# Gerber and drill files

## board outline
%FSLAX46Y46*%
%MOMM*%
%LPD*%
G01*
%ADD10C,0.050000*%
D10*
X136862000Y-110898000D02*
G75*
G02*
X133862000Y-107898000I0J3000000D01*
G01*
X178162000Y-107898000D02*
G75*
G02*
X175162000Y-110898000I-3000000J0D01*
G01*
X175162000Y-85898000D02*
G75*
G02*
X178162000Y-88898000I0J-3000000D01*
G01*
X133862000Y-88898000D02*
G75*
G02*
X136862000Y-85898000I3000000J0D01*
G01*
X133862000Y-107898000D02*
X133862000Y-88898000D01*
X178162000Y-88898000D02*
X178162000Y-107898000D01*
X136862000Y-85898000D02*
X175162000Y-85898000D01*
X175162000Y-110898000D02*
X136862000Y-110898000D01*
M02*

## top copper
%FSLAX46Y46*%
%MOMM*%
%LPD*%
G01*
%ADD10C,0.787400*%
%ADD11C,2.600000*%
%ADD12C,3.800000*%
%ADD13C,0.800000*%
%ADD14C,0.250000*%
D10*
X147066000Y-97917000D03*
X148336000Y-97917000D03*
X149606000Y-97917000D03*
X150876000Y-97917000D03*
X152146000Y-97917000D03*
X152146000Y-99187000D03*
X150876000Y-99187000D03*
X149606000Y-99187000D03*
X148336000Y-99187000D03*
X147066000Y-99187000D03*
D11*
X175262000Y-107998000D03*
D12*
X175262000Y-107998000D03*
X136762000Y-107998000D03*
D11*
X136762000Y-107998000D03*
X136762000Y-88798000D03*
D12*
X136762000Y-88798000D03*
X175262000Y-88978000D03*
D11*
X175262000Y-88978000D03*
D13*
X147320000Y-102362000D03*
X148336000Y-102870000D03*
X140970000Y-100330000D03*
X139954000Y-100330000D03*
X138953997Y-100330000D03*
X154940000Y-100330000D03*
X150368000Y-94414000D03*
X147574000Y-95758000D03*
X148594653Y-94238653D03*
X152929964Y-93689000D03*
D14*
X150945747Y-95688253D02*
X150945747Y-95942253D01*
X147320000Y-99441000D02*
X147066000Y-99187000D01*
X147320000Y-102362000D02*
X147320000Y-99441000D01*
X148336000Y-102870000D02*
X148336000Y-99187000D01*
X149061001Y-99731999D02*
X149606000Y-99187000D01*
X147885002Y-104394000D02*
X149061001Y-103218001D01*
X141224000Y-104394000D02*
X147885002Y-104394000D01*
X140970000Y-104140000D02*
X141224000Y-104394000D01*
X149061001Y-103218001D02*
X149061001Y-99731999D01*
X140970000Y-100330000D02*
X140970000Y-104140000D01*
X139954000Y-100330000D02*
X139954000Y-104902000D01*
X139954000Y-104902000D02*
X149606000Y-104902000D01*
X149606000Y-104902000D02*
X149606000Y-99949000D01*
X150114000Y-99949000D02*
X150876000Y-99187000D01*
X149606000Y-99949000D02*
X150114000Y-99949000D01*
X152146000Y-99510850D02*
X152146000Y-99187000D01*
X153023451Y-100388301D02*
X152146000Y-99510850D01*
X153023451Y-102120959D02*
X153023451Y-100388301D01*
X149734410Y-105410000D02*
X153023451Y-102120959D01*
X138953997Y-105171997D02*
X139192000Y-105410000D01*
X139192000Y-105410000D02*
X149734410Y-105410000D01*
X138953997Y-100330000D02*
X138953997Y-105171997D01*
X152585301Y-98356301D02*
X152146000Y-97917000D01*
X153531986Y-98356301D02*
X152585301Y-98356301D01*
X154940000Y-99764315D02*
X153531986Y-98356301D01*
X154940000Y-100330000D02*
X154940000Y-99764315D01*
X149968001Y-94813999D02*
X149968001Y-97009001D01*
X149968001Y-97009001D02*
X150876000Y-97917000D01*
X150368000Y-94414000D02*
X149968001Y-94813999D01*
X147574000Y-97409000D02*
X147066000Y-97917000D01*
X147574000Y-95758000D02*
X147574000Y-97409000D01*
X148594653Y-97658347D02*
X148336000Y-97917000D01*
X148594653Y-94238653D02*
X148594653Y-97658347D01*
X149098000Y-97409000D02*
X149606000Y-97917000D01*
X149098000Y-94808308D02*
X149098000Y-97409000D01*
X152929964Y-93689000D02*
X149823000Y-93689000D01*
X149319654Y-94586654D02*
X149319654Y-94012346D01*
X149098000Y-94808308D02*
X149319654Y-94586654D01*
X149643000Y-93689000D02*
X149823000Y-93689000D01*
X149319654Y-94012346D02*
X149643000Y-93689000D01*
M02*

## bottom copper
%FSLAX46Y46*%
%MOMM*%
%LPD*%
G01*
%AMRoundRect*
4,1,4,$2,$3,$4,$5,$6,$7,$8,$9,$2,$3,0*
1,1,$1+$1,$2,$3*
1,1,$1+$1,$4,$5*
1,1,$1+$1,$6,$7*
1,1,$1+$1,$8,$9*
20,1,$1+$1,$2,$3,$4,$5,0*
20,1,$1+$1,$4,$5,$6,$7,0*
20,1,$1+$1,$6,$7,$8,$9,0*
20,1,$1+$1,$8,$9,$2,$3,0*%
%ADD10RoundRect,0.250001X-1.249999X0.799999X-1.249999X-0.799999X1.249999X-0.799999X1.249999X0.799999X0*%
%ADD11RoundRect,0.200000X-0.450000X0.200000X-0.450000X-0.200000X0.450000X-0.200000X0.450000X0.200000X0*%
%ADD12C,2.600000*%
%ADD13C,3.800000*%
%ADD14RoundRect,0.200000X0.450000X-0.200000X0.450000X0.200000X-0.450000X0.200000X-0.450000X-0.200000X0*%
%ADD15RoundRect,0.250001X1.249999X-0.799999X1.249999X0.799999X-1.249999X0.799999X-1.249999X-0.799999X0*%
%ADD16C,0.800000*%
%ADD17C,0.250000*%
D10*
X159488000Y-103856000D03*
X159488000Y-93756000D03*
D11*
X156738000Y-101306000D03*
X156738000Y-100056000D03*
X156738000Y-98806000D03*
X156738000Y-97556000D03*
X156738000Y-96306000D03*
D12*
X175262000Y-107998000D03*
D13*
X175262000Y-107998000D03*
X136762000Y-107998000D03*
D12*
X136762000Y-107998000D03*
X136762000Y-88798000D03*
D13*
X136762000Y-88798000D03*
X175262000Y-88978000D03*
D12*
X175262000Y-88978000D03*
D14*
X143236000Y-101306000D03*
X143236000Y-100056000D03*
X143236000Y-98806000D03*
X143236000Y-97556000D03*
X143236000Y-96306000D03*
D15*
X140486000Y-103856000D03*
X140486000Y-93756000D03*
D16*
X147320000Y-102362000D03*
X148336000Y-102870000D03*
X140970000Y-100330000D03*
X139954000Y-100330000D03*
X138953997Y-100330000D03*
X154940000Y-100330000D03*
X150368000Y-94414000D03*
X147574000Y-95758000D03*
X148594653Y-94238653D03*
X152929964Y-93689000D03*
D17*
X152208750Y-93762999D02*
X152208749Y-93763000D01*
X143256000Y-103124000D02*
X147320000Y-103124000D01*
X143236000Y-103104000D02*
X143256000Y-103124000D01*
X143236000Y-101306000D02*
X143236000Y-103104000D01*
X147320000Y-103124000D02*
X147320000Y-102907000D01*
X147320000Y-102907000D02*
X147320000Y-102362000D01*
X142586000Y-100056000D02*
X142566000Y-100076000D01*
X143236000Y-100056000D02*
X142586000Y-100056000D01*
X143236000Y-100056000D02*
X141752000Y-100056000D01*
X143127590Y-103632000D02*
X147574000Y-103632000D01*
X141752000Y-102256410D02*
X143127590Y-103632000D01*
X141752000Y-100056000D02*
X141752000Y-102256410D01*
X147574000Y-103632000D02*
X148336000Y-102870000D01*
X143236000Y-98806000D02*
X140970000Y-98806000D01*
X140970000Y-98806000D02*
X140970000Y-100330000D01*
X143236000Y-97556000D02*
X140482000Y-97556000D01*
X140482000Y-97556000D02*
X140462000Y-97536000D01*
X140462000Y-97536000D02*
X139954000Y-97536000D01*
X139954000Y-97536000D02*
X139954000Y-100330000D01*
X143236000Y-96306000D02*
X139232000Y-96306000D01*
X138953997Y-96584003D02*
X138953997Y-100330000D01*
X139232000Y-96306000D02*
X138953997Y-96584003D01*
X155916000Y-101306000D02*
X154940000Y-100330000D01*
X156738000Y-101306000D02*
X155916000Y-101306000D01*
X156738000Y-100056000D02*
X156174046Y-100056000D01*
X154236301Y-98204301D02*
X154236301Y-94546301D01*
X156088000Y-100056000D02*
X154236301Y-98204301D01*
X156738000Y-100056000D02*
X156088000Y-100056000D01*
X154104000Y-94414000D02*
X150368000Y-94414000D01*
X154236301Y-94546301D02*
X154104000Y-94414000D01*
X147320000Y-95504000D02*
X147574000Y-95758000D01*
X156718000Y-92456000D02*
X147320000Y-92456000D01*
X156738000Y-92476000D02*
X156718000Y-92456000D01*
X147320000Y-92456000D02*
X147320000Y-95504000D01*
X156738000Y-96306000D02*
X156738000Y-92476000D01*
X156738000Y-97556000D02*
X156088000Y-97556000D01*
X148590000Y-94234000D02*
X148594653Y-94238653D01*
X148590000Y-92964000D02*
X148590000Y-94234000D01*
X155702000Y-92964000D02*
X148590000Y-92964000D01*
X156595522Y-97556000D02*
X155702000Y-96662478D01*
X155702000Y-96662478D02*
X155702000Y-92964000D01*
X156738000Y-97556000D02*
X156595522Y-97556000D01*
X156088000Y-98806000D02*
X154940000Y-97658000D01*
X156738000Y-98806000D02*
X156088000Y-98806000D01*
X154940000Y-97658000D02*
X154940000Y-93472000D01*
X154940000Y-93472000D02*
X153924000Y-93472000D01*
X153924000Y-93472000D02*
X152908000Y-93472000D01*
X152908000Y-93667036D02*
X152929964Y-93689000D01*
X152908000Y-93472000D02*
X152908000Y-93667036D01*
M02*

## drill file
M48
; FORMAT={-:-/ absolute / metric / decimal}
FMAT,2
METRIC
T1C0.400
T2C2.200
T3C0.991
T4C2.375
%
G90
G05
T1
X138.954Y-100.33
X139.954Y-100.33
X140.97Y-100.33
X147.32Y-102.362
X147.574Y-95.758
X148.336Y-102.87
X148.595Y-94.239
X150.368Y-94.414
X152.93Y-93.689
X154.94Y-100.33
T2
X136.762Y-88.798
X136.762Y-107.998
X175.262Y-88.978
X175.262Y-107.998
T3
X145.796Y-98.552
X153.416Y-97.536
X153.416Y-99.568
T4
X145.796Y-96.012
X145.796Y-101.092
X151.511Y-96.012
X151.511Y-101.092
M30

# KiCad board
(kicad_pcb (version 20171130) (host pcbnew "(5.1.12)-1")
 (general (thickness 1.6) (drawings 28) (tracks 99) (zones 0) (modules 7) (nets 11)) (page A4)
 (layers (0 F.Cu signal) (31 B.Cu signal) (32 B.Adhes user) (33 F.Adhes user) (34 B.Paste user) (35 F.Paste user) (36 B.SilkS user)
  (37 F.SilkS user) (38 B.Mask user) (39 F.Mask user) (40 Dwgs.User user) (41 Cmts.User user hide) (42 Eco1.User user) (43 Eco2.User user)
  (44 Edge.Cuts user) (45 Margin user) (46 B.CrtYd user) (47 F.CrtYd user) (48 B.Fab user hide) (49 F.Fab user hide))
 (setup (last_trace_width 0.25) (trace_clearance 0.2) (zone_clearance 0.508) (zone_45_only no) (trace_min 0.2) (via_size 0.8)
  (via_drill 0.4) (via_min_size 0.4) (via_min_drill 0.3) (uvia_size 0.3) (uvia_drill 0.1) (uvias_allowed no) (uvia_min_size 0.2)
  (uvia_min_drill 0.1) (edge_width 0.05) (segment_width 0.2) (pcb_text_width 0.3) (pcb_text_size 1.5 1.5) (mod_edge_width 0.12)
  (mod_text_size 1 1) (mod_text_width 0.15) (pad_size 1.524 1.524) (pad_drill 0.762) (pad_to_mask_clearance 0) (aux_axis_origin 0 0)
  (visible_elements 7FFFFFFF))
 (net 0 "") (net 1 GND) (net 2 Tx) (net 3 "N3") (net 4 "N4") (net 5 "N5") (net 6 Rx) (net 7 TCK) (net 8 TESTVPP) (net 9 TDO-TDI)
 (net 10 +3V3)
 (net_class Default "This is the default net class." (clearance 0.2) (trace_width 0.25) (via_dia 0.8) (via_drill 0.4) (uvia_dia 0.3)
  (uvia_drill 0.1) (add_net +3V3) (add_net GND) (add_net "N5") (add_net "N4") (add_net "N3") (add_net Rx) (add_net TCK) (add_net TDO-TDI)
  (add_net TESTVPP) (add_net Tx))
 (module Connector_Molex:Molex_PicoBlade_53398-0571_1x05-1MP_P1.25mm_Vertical (layer B.Cu) (at 157.988 98.806 270)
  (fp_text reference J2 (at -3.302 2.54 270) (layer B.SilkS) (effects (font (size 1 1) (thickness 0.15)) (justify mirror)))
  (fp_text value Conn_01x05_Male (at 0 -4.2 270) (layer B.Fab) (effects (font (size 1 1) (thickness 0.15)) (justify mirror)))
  (pad MP smd roundrect (at 5.05 -1.5 270) (size 2.1 3) (layers B.Cu B.Paste B.Mask) (roundrect_rratio 0.119048))
  (pad MP smd roundrect (at -5.05 -1.5 270) (size 2.1 3) (layers B.Cu B.Paste B.Mask) (roundrect_rratio 0.119048))
  (pad 5 smd roundrect (at 2.5 1.25 270) (size 0.8 1.3) (layers B.Cu B.Paste B.Mask) (roundrect_rratio 0.25) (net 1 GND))
  (pad 4 smd roundrect (at 1.25 1.25 270) (size 0.8 1.3) (layers B.Cu B.Paste B.Mask) (roundrect_rratio 0.25) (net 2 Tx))
  (pad 3 smd roundrect (at 0 1.25 270) (size 0.8 1.3) (layers B.Cu B.Paste B.Mask) (roundrect_rratio 0.25) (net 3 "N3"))
  (pad 2 smd roundrect (at -1.25 1.25 270) (size 0.8 1.3) (layers B.Cu B.Paste B.Mask) (roundrect_rratio 0.25) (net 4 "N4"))
  (pad 1 smd roundrect (at -2.5 1.25 270) (size 0.8 1.3) (layers B.Cu B.Paste B.Mask) (roundrect_rratio 0.25) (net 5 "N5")))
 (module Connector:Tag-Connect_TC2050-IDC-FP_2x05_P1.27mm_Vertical (layer F.Cu) (at 149.606 98.552)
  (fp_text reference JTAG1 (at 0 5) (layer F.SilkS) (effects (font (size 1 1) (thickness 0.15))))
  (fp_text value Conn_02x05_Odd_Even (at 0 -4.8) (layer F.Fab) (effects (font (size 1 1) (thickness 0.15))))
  (pad "" np_thru_hole circle (at 1.905 -2.54) (size 2.3749 2.3749) (drill 2.3749) (layers *.Cu *.Mask))
  (pad "" np_thru_hole circle (at 1.905 2.54) (size 2.3749 2.3749) (drill 2.3749) (layers *.Cu *.Mask))
  (pad "" np_thru_hole circle (at -3.81 2.54) (size 2.3749 2.3749) (drill 2.3749) (layers *.Cu *.Mask))
  (pad "" np_thru_hole circle (at -3.81 -2.54) (size 2.3749 2.3749) (drill 2.3749) (layers *.Cu *.Mask))
  (pad 10 connect circle (at -2.54 -0.635) (size 0.7874 0.7874) (layers F.Cu F.Mask) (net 5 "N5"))
  (pad 9 connect circle (at -1.27 -0.635) (size 0.7874 0.7874) (layers F.Cu F.Mask) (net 4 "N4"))
  (pad 8 connect circle (at 0 -0.635) (size 0.7874 0.7874) (layers F.Cu F.Mask) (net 3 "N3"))
  (pad 7 connect circle (at 1.27 -0.635) (size 0.7874 0.7874) (layers F.Cu F.Mask) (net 2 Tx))
  (pad 6 connect circle (at 2.54 -0.635) (size 0.7874 0.7874) (layers F.Cu F.Mask) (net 1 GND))
  (pad 5 connect circle (at 2.54 0.635) (size 0.7874 0.7874) (layers F.Cu F.Mask) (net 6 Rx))
  (pad 4 connect circle (at 1.27 0.635) (size 0.7874 0.7874) (layers F.Cu F.Mask) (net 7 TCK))
  (pad 3 connect circle (at 0 0.635) (size 0.7874 0.7874) (layers F.Cu F.Mask) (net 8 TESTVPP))
  (pad 2 connect circle (at -1.27 0.635) (size 0.7874 0.7874) (layers F.Cu F.Mask) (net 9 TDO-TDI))
  (pad 1 connect circle (at -2.54 0.635) (size 0.7874 0.7874) (layers F.Cu F.Mask) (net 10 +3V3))
  (pad "" np_thru_hole circle (at -3.81 0) (size 0.9906 0.9906) (drill 0.9906) (layers *.Cu *.Mask))
  (pad "" np_thru_hole circle (at 3.81 1.016) (size 0.9906 0.9906) (drill 0.9906) (layers *.Cu *.Mask))
  (pad "" np_thru_hole circle (at 3.81 -1.016) (size 0.9906 0.9906) (drill 0.9906) (layers *.Cu *.Mask)))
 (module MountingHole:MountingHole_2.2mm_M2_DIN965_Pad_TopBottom (layer F.Cu) (at 175.262 107.998)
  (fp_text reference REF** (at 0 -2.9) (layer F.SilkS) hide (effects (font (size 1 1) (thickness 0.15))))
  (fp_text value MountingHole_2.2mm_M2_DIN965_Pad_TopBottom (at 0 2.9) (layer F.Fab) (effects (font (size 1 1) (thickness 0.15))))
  (pad 1 thru_hole circle (at 0 0) (size 2.6 2.6) (drill 2.2) (layers *.Cu *.Mask))
  (pad 1 connect circle (at 0 0) (size 3.8 3.8) (layers F.Cu F.Mask))
  (pad 1 connect circle (at 0 0) (size 3.8 3.8) (layers B.Cu B.Mask)))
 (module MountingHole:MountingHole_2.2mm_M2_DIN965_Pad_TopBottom (layer F.Cu) (at 136.762 107.998)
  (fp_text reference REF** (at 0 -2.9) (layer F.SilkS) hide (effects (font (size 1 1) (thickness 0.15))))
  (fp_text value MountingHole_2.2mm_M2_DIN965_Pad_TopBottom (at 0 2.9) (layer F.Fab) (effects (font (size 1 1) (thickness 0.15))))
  (pad 1 connect circle (at 0 0) (size 3.8 3.8) (layers B.Cu B.Mask))
  (pad 1 connect circle (at 0 0) (size 3.8 3.8) (layers F.Cu F.Mask))
  (pad 1 thru_hole circle (at 0 0) (size 2.6 2.6) (drill 2.2) (layers *.Cu *.Mask)))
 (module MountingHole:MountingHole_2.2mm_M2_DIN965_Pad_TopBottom (layer F.Cu) (at 136.762 88.798)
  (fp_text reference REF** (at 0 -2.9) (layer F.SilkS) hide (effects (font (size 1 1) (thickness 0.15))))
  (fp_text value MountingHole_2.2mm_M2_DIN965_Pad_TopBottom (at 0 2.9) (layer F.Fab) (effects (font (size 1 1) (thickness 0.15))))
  (pad 1 thru_hole circle (at 0 0) (size 2.6 2.6) (drill 2.2) (layers *.Cu *.Mask))
  (pad 1 connect circle (at 0 0) (size 3.8 3.8) (layers F.Cu F.Mask))
  (pad 1 connect circle (at 0 0) (size 3.8 3.8) (layers B.Cu B.Mask)))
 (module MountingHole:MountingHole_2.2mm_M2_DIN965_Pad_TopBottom (layer F.Cu) (at 175.262 88.978)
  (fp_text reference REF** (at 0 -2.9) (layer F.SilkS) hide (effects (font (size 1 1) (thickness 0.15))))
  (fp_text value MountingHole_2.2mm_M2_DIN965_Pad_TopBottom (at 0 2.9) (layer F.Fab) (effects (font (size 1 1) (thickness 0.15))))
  (pad 1 connect circle (at 0 0) (size 3.8 3.8) (layers B.Cu B.Mask))
  (pad 1 connect circle (at 0 0) (size 3.8 3.8) (layers F.Cu F.Mask))
  (pad 1 thru_hole circle (at 0 0) (size 2.6 2.6) (drill 2.2) (layers *.Cu *.Mask)))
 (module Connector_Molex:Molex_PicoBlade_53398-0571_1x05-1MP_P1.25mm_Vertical (layer B.Cu) (at 141.986 98.806 90)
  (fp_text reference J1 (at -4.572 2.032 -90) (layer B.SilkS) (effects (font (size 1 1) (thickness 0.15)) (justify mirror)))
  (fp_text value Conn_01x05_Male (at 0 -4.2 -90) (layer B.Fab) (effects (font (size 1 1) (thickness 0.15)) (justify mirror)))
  (pad 1 smd roundrect (at -2.5 1.25 90) (size 0.8 1.3) (layers B.Cu B.Paste B.Mask) (roundrect_rratio 0.25) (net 10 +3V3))
  (pad 2 smd roundrect (at -1.25 1.25 90) (size 0.8 1.3) (layers B.Cu B.Paste B.Mask) (roundrect_rratio 0.25) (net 9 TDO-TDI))
  (pad 3 smd roundrect (at 0 1.25 90) (size 0.8 1.3) (layers B.Cu B.Paste B.Mask) (roundrect_rratio 0.25) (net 8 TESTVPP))
  (pad 4 smd roundrect (at 1.25 1.25 90) (size 0.8 1.3) (layers B.Cu B.Paste B.Mask) (roundrect_rratio 0.25) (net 7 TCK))
  (pad 5 smd roundrect (at 2.5 1.25 90) (size 0.8 1.3) (layers B.Cu B.Paste B.Mask) (roundrect_rratio 0.25) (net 6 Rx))
  (pad MP smd roundrect (at -5.05 -1.5 90) (size 2.1 3) (layers B.Cu B.Paste B.Mask) (roundrect_rratio 0.119048))
  (pad MP smd roundrect (at 5.05 -1.5 90) (size 2.1 3) (layers B.Cu B.Paste B.Mask) (roundrect_rratio 0.119048)))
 (gr_arc (start 136.862 107.898) (end 133.862 107.898) (angle -90) (layer Edge.Cuts) (width 0.05))
 (gr_arc (start 175.162 107.898) (end 175.162 110.898) (angle -90) (layer Edge.Cuts) (width 0.05))
 (gr_arc (start 175.162 88.898) (end 178.162 88.898) (angle -90) (layer Edge.Cuts) (width 0.05))
 (gr_arc (start 136.862 88.898) (end 136.862 85.898) (angle -90) (layer Edge.Cuts) (width 0.05))
 (gr_line (start 133.862 107.898) (end 133.862 88.898) (layer Edge.Cuts) (width 0.05))
 (gr_line (start 178.162 88.898) (end 178.162 107.898) (layer Edge.Cuts) (width 0.05))
 (gr_line (start 136.862 85.898) (end 175.162 85.898) (layer Edge.Cuts) (width 0.05))
 (gr_line (start 175.162 110.898) (end 136.862 110.898) (layer Edge.Cuts) (width 0.05))
 (segment (start 150.945747 95.688253) (end 150.945747 95.942253) (width 0.25) (layer F.Cu) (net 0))
 (segment (start 152.20875 93.762999) (end 152.208749 93.763) (width 0.25) (layer B.Cu) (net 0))
 (segment (start 143.256 103.124) (end 147.32 103.124) (width 0.25) (layer B.Cu) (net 10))
 (segment (start 143.236 103.104) (end 143.256 103.124) (width 0.25) (layer B.Cu) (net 10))
 (segment (start 143.236 101.306) (end 143.236 103.104) (width 0.25) (layer B.Cu) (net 10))
 (segment (start 147.32 103.124) (end 147.32 102.907) (width 0.25) (layer B.Cu) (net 10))
 (via (at 147.32 102.362) (size 0.8) (drill 0.4) (layers F.Cu B.Cu) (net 10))
 (segment (start 147.32 102.907) (end 147.32 102.362) (width 0.25) (layer B.Cu) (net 10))
 (segment (start 147.32 99.441) (end 147.066 99.187) (width 0.25) (layer F.Cu) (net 10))
 (segment (start 147.32 102.362) (end 147.32 99.441) (width 0.25) (layer F.Cu) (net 10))
 (segment (start 142.586 100.056) (end 142.566 100.076) (width 0.25) (layer B.Cu) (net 9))
 (segment (start 143.236 100.056) (end 142.586 100.056) (width 0.25) (layer B.Cu) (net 9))
 (segment (start 143.236 100.056) (end 141.752 100.056) (width 0.25) (layer B.Cu) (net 9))
 (segment (start 143.12759 103.632) (end 147.574 103.632) (width 0.25) (layer B.Cu) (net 9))
 (segment (start 141.752 102.25641) (end 143.12759 103.632) (width 0.25) (layer B.Cu) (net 9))
 (segment (start 141.752 100.056) (end 141.752 102.25641) (width 0.25) (layer B.Cu) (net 9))
 (via (at 148.336 102.87) (size 0.8) (drill 0.4) (layers F.Cu B.Cu) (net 9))
 (segment (start 147.574 103.632) (end 148.336 102.87) (width 0.25) (layer B.Cu) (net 9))
 (segment (start 148.336 102.87) (end 148.336 99.187) (width 0.25) (layer F.Cu) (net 9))
 (segment (start 143.236 98.806) (end 140.97 98.806) (width 0.25) (layer B.Cu) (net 8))
 (via (at 140.97 100.33) (size 0.8) (drill 0.4) (layers F.Cu B.Cu) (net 8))
 (segment (start 140.97 98.806) (end 140.97 100.33) (width 0.25) (layer B.Cu) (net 8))
 (segment (start 149.061001 99.731999) (end 149.606 99.187) (width 0.25) (layer F.Cu) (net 8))
 (segment (start 147.885002 104.394) (end 149.061001 103.218001) (width 0.25) (layer F.Cu) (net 8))
 (segment (start 141.224 104.394) (end 147.885002 104.394) (width 0.25) (layer F.Cu) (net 8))
 (segment (start 140.97 104.14) (end 141.224 104.394) (width 0.25) (layer F.Cu) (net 8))
 (segment (start 149.061001 103.218001) (end 149.061001 99.731999) (width 0.25) (layer F.Cu) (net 8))
 (segment (start 140.97 100.33) (end 140.97 104.14) (width 0.25) (layer F.Cu) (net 8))
 (segment (start 143.236 97.556) (end 140.482 97.556) (width 0.25) (layer B.Cu) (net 7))
 (segment (start 140.482 97.556) (end 140.462 97.536) (width 0.25) (layer B.Cu) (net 7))
 (segment (start 140.462 97.536) (end 139.954 97.536) (width 0.25) (layer B.Cu) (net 7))
 (via (at 139.954 100.33) (size 0.8) (drill 0.4) (layers F.Cu B.Cu) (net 7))
 (segment (start 139.954 97.536) (end 139.954 100.33) (width 0.25) (layer B.Cu) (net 7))
 (segment (start 139.954 100.33) (end 139.954 104.902) (width 0.25) (layer F.Cu) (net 7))
 (segment (start 139.954 104.902) (end 149.606 104.902) (width 0.25) (layer F.Cu) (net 7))
 (segment (start 149.606 104.902) (end 149.606 99.949) (width 0.25) (layer F.Cu) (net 7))
 (segment (start 150.114 99.949) (end 150.876 99.187) (width 0.25) (layer F.Cu) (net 7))
 (segment (start 149.606 99.949) (end 150.114 99.949) (width 0.25) (layer F.Cu) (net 7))
 (segment (start 143.236 96.306) (end 139.232 96.306) (width 0.25) (layer B.Cu) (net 6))
 (via (at 138.953997 100.33) (size 0.8) (drill 0.4) (layers F.Cu B.Cu) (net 6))
 (segment (start 138.953997 96.584003) (end 138.953997 100.33) (width 0.25) (layer B.Cu) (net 6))
 (segment (start 139.232 96.306) (end 138.953997 96.584003) (width 0.25) (layer B.Cu) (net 6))
 (segment (start 152.146 99.51085) (end 152.146 99.187) (width 0.25) (layer F.Cu) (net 6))
 (segment (start 153.023451 100.388301) (end 152.146 99.51085) (width 0.25) (layer F.Cu) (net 6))
 (segment (start 153.023451 102.120959) (end 153.023451 100.388301) (width 0.25) (layer F.Cu) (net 6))
 (segment (start 149.73441 105.41) (end 153.023451 102.120959) (width 0.25) (layer F.Cu) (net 6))
 (segment (start 138.953997 105.171997) (end 139.192 105.41) (width 0.25) (layer F.Cu) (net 6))
 (segment (start 139.192 105.41) (end 149.73441 105.41) (width 0.25) (layer F.Cu) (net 6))
 (segment (start 138.953997 100.33) (end 138.953997 105.171997) (width 0.25) (layer F.Cu) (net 6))
 (via (at 154.94 100.33) (size 0.8) (drill 0.4) (layers F.Cu B.Cu) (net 1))
 (segment (start 155.916 101.306) (end 154.94 100.33) (width 0.25) (layer B.Cu) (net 1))
 (segment (start 156.738 101.306) (end 155.916 101.306) (width 0.25) (layer B.Cu) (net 1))
 (segment (start 152.585301 98.356301) (end 152.146 97.917) (width 0.25) (layer F.Cu) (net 1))
 (segment (start 153.531986 98.356301) (end 152.585301 98.356301) (width 0.25) (layer F.Cu) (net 1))
 (segment (start 154.94 99.764315) (end 153.531986 98.356301) (width 0.25) (layer F.Cu) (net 1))
 (segment (start 154.94 100.33) (end 154.94 99.764315) (width 0.25) (layer F.Cu) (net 1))
 (segment (start 156.738 100.056) (end 156.174046 100.056) (width 0.25) (layer B.Cu) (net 2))
 (segment (start 154.236301 98.204301) (end 154.236301 94.546301) (width 0.25) (layer B.Cu) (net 2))
 (segment (start 156.088 100.056) (end 154.236301 98.204301) (width 0.25) (layer B.Cu) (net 2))
 (segment (start 156.738 100.056) (end 156.088 100.056) (width 0.25) (layer B.Cu) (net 2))
 (segment (start 154.104 94.414) (end 150.368 94.414) (width 0.25) (layer B.Cu) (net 2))
 (via (at 150.368 94.414) (size 0.8) (drill 0.4) (layers F.Cu B.Cu) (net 2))
 (segment (start 154.236301 94.546301) (end 154.104 94.414) (width 0.25) (layer B.Cu) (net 2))
 (segment (start 149.968001 94.813999) (end 149.968001 97.009001) (width 0.25) (layer F.Cu) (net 2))
 (segment (start 149.968001 97.009001) (end 150.876 97.917) (width 0.25) (layer F.Cu) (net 2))
 (segment (start 150.368 94.414) (end 149.968001 94.813999) (width 0.25) (layer F.Cu) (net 2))
 (via (at 147.574 95.758) (size 0.8) (drill 0.4) (layers F.Cu B.Cu) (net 5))
 (segment (start 147.574 97.409) (end 147.066 97.917) (width 0.25) (layer F.Cu) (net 5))
 (segment (start 147.574 95.758) (end 147.574 97.409) (width 0.25) (layer F.Cu) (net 5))
 (segment (start 147.32 95.504) (end 147.574 95.758) (width 0.25) (layer B.Cu) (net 5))
 (segment (start 156.718 92.456) (end 147.32 92.456) (width 0.25) (layer B.Cu) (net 5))
 (segment (start 156.738 92.476) (end 156.718 92.456) (width 0.25) (layer B.Cu) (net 5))
 (segment (start 147.32 92.456) (end 147.32 95.504) (width 0.25) (layer B.Cu) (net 5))
 (segment (start 156.738 96.306) (end 156.738 92.476) (width 0.25) (layer B.Cu) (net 5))
 (segment (start 156.738 97.556) (end 156.088 97.556) (width 0.25) (layer B.Cu) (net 4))
 (via (at 148.594653 94.238653) (size 0.8) (drill 0.4) (layers F.Cu B.Cu) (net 4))
 (segment (start 148.594653 97.658347) (end 148.336 97.917) (width 0.25) (layer F.Cu) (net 4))
 (segment (start 148.594653 94.238653) (end 148.594653 97.658347) (width 0.25) (layer F.Cu) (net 4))
 (segment (start 148.59 94.234) (end 148.594653 94.238653) (width 0.25) (layer B.Cu) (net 4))
 (segment (start 148.59 92.964) (end 148.59 94.234) (width 0.25) (layer B.Cu) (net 4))
 (segment (start 155.702 92.964) (end 148.59 92.964) (width 0.25) (layer B.Cu) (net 4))
 (segment (start 156.595522 97.556) (end 155.702 96.662478) (width 0.25) (layer B.Cu) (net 4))
 (segment (start 155.702 96.662478) (end 155.702 92.964) (width 0.25) (layer B.Cu) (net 4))
 (segment (start 156.738 97.556) (end 156.595522 97.556) (width 0.25) (layer B.Cu) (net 4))
 (segment (start 156.088 98.806) (end 154.94 97.658) (width 0.25) (layer B.Cu) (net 3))
 (segment (start 156.738 98.806) (end 156.088 98.806) (width 0.25) (layer B.Cu) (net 3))
 (segment (start 154.94 97.658) (end 154.94 93.472) (width 0.25) (layer B.Cu) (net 3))
 (segment (start 154.94 93.472) (end 153.924 93.472) (width 0.25) (layer B.Cu) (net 3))
 (segment (start 153.924 93.472) (end 152.908 93.472) (width 0.25) (layer B.Cu) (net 3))
 (via (at 152.929964 93.689) (size 0.8) (drill 0.4) (layers F.Cu B.Cu) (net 3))
 (segment (start 152.908 93.667036) (end 152.929964 93.689) (width 0.25) (layer B.Cu) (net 3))
 (segment (start 152.908 93.472) (end 152.908 93.667036) (width 0.25) (layer B.Cu) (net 3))
 (segment (start 149.098 97.409) (end 149.606 97.917) (width 0.25) (layer F.Cu) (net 3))
 (segment (start 149.098 94.808308) (end 149.098 97.409) (width 0.25) (layer F.Cu) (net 3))
 (segment (start 152.929964 93.689) (end 149.823 93.689) (width 0.25) (layer F.Cu) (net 3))
 (segment (start 149.319654 94.586654) (end 149.319654 94.012346) (width 0.25) (layer F.Cu) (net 3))
 (segment (start 149.098 94.808308) (end 149.319654 94.586654) (width 0.25) (layer F.Cu) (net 3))
 (segment (start 149.643 93.689) (end 149.823 93.689) (width 0.25) (layer F.Cu) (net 3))
 (segment (start 149.319654 94.012346) (end 149.643 93.689) (width 0.25) (layer F.Cu) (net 3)))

